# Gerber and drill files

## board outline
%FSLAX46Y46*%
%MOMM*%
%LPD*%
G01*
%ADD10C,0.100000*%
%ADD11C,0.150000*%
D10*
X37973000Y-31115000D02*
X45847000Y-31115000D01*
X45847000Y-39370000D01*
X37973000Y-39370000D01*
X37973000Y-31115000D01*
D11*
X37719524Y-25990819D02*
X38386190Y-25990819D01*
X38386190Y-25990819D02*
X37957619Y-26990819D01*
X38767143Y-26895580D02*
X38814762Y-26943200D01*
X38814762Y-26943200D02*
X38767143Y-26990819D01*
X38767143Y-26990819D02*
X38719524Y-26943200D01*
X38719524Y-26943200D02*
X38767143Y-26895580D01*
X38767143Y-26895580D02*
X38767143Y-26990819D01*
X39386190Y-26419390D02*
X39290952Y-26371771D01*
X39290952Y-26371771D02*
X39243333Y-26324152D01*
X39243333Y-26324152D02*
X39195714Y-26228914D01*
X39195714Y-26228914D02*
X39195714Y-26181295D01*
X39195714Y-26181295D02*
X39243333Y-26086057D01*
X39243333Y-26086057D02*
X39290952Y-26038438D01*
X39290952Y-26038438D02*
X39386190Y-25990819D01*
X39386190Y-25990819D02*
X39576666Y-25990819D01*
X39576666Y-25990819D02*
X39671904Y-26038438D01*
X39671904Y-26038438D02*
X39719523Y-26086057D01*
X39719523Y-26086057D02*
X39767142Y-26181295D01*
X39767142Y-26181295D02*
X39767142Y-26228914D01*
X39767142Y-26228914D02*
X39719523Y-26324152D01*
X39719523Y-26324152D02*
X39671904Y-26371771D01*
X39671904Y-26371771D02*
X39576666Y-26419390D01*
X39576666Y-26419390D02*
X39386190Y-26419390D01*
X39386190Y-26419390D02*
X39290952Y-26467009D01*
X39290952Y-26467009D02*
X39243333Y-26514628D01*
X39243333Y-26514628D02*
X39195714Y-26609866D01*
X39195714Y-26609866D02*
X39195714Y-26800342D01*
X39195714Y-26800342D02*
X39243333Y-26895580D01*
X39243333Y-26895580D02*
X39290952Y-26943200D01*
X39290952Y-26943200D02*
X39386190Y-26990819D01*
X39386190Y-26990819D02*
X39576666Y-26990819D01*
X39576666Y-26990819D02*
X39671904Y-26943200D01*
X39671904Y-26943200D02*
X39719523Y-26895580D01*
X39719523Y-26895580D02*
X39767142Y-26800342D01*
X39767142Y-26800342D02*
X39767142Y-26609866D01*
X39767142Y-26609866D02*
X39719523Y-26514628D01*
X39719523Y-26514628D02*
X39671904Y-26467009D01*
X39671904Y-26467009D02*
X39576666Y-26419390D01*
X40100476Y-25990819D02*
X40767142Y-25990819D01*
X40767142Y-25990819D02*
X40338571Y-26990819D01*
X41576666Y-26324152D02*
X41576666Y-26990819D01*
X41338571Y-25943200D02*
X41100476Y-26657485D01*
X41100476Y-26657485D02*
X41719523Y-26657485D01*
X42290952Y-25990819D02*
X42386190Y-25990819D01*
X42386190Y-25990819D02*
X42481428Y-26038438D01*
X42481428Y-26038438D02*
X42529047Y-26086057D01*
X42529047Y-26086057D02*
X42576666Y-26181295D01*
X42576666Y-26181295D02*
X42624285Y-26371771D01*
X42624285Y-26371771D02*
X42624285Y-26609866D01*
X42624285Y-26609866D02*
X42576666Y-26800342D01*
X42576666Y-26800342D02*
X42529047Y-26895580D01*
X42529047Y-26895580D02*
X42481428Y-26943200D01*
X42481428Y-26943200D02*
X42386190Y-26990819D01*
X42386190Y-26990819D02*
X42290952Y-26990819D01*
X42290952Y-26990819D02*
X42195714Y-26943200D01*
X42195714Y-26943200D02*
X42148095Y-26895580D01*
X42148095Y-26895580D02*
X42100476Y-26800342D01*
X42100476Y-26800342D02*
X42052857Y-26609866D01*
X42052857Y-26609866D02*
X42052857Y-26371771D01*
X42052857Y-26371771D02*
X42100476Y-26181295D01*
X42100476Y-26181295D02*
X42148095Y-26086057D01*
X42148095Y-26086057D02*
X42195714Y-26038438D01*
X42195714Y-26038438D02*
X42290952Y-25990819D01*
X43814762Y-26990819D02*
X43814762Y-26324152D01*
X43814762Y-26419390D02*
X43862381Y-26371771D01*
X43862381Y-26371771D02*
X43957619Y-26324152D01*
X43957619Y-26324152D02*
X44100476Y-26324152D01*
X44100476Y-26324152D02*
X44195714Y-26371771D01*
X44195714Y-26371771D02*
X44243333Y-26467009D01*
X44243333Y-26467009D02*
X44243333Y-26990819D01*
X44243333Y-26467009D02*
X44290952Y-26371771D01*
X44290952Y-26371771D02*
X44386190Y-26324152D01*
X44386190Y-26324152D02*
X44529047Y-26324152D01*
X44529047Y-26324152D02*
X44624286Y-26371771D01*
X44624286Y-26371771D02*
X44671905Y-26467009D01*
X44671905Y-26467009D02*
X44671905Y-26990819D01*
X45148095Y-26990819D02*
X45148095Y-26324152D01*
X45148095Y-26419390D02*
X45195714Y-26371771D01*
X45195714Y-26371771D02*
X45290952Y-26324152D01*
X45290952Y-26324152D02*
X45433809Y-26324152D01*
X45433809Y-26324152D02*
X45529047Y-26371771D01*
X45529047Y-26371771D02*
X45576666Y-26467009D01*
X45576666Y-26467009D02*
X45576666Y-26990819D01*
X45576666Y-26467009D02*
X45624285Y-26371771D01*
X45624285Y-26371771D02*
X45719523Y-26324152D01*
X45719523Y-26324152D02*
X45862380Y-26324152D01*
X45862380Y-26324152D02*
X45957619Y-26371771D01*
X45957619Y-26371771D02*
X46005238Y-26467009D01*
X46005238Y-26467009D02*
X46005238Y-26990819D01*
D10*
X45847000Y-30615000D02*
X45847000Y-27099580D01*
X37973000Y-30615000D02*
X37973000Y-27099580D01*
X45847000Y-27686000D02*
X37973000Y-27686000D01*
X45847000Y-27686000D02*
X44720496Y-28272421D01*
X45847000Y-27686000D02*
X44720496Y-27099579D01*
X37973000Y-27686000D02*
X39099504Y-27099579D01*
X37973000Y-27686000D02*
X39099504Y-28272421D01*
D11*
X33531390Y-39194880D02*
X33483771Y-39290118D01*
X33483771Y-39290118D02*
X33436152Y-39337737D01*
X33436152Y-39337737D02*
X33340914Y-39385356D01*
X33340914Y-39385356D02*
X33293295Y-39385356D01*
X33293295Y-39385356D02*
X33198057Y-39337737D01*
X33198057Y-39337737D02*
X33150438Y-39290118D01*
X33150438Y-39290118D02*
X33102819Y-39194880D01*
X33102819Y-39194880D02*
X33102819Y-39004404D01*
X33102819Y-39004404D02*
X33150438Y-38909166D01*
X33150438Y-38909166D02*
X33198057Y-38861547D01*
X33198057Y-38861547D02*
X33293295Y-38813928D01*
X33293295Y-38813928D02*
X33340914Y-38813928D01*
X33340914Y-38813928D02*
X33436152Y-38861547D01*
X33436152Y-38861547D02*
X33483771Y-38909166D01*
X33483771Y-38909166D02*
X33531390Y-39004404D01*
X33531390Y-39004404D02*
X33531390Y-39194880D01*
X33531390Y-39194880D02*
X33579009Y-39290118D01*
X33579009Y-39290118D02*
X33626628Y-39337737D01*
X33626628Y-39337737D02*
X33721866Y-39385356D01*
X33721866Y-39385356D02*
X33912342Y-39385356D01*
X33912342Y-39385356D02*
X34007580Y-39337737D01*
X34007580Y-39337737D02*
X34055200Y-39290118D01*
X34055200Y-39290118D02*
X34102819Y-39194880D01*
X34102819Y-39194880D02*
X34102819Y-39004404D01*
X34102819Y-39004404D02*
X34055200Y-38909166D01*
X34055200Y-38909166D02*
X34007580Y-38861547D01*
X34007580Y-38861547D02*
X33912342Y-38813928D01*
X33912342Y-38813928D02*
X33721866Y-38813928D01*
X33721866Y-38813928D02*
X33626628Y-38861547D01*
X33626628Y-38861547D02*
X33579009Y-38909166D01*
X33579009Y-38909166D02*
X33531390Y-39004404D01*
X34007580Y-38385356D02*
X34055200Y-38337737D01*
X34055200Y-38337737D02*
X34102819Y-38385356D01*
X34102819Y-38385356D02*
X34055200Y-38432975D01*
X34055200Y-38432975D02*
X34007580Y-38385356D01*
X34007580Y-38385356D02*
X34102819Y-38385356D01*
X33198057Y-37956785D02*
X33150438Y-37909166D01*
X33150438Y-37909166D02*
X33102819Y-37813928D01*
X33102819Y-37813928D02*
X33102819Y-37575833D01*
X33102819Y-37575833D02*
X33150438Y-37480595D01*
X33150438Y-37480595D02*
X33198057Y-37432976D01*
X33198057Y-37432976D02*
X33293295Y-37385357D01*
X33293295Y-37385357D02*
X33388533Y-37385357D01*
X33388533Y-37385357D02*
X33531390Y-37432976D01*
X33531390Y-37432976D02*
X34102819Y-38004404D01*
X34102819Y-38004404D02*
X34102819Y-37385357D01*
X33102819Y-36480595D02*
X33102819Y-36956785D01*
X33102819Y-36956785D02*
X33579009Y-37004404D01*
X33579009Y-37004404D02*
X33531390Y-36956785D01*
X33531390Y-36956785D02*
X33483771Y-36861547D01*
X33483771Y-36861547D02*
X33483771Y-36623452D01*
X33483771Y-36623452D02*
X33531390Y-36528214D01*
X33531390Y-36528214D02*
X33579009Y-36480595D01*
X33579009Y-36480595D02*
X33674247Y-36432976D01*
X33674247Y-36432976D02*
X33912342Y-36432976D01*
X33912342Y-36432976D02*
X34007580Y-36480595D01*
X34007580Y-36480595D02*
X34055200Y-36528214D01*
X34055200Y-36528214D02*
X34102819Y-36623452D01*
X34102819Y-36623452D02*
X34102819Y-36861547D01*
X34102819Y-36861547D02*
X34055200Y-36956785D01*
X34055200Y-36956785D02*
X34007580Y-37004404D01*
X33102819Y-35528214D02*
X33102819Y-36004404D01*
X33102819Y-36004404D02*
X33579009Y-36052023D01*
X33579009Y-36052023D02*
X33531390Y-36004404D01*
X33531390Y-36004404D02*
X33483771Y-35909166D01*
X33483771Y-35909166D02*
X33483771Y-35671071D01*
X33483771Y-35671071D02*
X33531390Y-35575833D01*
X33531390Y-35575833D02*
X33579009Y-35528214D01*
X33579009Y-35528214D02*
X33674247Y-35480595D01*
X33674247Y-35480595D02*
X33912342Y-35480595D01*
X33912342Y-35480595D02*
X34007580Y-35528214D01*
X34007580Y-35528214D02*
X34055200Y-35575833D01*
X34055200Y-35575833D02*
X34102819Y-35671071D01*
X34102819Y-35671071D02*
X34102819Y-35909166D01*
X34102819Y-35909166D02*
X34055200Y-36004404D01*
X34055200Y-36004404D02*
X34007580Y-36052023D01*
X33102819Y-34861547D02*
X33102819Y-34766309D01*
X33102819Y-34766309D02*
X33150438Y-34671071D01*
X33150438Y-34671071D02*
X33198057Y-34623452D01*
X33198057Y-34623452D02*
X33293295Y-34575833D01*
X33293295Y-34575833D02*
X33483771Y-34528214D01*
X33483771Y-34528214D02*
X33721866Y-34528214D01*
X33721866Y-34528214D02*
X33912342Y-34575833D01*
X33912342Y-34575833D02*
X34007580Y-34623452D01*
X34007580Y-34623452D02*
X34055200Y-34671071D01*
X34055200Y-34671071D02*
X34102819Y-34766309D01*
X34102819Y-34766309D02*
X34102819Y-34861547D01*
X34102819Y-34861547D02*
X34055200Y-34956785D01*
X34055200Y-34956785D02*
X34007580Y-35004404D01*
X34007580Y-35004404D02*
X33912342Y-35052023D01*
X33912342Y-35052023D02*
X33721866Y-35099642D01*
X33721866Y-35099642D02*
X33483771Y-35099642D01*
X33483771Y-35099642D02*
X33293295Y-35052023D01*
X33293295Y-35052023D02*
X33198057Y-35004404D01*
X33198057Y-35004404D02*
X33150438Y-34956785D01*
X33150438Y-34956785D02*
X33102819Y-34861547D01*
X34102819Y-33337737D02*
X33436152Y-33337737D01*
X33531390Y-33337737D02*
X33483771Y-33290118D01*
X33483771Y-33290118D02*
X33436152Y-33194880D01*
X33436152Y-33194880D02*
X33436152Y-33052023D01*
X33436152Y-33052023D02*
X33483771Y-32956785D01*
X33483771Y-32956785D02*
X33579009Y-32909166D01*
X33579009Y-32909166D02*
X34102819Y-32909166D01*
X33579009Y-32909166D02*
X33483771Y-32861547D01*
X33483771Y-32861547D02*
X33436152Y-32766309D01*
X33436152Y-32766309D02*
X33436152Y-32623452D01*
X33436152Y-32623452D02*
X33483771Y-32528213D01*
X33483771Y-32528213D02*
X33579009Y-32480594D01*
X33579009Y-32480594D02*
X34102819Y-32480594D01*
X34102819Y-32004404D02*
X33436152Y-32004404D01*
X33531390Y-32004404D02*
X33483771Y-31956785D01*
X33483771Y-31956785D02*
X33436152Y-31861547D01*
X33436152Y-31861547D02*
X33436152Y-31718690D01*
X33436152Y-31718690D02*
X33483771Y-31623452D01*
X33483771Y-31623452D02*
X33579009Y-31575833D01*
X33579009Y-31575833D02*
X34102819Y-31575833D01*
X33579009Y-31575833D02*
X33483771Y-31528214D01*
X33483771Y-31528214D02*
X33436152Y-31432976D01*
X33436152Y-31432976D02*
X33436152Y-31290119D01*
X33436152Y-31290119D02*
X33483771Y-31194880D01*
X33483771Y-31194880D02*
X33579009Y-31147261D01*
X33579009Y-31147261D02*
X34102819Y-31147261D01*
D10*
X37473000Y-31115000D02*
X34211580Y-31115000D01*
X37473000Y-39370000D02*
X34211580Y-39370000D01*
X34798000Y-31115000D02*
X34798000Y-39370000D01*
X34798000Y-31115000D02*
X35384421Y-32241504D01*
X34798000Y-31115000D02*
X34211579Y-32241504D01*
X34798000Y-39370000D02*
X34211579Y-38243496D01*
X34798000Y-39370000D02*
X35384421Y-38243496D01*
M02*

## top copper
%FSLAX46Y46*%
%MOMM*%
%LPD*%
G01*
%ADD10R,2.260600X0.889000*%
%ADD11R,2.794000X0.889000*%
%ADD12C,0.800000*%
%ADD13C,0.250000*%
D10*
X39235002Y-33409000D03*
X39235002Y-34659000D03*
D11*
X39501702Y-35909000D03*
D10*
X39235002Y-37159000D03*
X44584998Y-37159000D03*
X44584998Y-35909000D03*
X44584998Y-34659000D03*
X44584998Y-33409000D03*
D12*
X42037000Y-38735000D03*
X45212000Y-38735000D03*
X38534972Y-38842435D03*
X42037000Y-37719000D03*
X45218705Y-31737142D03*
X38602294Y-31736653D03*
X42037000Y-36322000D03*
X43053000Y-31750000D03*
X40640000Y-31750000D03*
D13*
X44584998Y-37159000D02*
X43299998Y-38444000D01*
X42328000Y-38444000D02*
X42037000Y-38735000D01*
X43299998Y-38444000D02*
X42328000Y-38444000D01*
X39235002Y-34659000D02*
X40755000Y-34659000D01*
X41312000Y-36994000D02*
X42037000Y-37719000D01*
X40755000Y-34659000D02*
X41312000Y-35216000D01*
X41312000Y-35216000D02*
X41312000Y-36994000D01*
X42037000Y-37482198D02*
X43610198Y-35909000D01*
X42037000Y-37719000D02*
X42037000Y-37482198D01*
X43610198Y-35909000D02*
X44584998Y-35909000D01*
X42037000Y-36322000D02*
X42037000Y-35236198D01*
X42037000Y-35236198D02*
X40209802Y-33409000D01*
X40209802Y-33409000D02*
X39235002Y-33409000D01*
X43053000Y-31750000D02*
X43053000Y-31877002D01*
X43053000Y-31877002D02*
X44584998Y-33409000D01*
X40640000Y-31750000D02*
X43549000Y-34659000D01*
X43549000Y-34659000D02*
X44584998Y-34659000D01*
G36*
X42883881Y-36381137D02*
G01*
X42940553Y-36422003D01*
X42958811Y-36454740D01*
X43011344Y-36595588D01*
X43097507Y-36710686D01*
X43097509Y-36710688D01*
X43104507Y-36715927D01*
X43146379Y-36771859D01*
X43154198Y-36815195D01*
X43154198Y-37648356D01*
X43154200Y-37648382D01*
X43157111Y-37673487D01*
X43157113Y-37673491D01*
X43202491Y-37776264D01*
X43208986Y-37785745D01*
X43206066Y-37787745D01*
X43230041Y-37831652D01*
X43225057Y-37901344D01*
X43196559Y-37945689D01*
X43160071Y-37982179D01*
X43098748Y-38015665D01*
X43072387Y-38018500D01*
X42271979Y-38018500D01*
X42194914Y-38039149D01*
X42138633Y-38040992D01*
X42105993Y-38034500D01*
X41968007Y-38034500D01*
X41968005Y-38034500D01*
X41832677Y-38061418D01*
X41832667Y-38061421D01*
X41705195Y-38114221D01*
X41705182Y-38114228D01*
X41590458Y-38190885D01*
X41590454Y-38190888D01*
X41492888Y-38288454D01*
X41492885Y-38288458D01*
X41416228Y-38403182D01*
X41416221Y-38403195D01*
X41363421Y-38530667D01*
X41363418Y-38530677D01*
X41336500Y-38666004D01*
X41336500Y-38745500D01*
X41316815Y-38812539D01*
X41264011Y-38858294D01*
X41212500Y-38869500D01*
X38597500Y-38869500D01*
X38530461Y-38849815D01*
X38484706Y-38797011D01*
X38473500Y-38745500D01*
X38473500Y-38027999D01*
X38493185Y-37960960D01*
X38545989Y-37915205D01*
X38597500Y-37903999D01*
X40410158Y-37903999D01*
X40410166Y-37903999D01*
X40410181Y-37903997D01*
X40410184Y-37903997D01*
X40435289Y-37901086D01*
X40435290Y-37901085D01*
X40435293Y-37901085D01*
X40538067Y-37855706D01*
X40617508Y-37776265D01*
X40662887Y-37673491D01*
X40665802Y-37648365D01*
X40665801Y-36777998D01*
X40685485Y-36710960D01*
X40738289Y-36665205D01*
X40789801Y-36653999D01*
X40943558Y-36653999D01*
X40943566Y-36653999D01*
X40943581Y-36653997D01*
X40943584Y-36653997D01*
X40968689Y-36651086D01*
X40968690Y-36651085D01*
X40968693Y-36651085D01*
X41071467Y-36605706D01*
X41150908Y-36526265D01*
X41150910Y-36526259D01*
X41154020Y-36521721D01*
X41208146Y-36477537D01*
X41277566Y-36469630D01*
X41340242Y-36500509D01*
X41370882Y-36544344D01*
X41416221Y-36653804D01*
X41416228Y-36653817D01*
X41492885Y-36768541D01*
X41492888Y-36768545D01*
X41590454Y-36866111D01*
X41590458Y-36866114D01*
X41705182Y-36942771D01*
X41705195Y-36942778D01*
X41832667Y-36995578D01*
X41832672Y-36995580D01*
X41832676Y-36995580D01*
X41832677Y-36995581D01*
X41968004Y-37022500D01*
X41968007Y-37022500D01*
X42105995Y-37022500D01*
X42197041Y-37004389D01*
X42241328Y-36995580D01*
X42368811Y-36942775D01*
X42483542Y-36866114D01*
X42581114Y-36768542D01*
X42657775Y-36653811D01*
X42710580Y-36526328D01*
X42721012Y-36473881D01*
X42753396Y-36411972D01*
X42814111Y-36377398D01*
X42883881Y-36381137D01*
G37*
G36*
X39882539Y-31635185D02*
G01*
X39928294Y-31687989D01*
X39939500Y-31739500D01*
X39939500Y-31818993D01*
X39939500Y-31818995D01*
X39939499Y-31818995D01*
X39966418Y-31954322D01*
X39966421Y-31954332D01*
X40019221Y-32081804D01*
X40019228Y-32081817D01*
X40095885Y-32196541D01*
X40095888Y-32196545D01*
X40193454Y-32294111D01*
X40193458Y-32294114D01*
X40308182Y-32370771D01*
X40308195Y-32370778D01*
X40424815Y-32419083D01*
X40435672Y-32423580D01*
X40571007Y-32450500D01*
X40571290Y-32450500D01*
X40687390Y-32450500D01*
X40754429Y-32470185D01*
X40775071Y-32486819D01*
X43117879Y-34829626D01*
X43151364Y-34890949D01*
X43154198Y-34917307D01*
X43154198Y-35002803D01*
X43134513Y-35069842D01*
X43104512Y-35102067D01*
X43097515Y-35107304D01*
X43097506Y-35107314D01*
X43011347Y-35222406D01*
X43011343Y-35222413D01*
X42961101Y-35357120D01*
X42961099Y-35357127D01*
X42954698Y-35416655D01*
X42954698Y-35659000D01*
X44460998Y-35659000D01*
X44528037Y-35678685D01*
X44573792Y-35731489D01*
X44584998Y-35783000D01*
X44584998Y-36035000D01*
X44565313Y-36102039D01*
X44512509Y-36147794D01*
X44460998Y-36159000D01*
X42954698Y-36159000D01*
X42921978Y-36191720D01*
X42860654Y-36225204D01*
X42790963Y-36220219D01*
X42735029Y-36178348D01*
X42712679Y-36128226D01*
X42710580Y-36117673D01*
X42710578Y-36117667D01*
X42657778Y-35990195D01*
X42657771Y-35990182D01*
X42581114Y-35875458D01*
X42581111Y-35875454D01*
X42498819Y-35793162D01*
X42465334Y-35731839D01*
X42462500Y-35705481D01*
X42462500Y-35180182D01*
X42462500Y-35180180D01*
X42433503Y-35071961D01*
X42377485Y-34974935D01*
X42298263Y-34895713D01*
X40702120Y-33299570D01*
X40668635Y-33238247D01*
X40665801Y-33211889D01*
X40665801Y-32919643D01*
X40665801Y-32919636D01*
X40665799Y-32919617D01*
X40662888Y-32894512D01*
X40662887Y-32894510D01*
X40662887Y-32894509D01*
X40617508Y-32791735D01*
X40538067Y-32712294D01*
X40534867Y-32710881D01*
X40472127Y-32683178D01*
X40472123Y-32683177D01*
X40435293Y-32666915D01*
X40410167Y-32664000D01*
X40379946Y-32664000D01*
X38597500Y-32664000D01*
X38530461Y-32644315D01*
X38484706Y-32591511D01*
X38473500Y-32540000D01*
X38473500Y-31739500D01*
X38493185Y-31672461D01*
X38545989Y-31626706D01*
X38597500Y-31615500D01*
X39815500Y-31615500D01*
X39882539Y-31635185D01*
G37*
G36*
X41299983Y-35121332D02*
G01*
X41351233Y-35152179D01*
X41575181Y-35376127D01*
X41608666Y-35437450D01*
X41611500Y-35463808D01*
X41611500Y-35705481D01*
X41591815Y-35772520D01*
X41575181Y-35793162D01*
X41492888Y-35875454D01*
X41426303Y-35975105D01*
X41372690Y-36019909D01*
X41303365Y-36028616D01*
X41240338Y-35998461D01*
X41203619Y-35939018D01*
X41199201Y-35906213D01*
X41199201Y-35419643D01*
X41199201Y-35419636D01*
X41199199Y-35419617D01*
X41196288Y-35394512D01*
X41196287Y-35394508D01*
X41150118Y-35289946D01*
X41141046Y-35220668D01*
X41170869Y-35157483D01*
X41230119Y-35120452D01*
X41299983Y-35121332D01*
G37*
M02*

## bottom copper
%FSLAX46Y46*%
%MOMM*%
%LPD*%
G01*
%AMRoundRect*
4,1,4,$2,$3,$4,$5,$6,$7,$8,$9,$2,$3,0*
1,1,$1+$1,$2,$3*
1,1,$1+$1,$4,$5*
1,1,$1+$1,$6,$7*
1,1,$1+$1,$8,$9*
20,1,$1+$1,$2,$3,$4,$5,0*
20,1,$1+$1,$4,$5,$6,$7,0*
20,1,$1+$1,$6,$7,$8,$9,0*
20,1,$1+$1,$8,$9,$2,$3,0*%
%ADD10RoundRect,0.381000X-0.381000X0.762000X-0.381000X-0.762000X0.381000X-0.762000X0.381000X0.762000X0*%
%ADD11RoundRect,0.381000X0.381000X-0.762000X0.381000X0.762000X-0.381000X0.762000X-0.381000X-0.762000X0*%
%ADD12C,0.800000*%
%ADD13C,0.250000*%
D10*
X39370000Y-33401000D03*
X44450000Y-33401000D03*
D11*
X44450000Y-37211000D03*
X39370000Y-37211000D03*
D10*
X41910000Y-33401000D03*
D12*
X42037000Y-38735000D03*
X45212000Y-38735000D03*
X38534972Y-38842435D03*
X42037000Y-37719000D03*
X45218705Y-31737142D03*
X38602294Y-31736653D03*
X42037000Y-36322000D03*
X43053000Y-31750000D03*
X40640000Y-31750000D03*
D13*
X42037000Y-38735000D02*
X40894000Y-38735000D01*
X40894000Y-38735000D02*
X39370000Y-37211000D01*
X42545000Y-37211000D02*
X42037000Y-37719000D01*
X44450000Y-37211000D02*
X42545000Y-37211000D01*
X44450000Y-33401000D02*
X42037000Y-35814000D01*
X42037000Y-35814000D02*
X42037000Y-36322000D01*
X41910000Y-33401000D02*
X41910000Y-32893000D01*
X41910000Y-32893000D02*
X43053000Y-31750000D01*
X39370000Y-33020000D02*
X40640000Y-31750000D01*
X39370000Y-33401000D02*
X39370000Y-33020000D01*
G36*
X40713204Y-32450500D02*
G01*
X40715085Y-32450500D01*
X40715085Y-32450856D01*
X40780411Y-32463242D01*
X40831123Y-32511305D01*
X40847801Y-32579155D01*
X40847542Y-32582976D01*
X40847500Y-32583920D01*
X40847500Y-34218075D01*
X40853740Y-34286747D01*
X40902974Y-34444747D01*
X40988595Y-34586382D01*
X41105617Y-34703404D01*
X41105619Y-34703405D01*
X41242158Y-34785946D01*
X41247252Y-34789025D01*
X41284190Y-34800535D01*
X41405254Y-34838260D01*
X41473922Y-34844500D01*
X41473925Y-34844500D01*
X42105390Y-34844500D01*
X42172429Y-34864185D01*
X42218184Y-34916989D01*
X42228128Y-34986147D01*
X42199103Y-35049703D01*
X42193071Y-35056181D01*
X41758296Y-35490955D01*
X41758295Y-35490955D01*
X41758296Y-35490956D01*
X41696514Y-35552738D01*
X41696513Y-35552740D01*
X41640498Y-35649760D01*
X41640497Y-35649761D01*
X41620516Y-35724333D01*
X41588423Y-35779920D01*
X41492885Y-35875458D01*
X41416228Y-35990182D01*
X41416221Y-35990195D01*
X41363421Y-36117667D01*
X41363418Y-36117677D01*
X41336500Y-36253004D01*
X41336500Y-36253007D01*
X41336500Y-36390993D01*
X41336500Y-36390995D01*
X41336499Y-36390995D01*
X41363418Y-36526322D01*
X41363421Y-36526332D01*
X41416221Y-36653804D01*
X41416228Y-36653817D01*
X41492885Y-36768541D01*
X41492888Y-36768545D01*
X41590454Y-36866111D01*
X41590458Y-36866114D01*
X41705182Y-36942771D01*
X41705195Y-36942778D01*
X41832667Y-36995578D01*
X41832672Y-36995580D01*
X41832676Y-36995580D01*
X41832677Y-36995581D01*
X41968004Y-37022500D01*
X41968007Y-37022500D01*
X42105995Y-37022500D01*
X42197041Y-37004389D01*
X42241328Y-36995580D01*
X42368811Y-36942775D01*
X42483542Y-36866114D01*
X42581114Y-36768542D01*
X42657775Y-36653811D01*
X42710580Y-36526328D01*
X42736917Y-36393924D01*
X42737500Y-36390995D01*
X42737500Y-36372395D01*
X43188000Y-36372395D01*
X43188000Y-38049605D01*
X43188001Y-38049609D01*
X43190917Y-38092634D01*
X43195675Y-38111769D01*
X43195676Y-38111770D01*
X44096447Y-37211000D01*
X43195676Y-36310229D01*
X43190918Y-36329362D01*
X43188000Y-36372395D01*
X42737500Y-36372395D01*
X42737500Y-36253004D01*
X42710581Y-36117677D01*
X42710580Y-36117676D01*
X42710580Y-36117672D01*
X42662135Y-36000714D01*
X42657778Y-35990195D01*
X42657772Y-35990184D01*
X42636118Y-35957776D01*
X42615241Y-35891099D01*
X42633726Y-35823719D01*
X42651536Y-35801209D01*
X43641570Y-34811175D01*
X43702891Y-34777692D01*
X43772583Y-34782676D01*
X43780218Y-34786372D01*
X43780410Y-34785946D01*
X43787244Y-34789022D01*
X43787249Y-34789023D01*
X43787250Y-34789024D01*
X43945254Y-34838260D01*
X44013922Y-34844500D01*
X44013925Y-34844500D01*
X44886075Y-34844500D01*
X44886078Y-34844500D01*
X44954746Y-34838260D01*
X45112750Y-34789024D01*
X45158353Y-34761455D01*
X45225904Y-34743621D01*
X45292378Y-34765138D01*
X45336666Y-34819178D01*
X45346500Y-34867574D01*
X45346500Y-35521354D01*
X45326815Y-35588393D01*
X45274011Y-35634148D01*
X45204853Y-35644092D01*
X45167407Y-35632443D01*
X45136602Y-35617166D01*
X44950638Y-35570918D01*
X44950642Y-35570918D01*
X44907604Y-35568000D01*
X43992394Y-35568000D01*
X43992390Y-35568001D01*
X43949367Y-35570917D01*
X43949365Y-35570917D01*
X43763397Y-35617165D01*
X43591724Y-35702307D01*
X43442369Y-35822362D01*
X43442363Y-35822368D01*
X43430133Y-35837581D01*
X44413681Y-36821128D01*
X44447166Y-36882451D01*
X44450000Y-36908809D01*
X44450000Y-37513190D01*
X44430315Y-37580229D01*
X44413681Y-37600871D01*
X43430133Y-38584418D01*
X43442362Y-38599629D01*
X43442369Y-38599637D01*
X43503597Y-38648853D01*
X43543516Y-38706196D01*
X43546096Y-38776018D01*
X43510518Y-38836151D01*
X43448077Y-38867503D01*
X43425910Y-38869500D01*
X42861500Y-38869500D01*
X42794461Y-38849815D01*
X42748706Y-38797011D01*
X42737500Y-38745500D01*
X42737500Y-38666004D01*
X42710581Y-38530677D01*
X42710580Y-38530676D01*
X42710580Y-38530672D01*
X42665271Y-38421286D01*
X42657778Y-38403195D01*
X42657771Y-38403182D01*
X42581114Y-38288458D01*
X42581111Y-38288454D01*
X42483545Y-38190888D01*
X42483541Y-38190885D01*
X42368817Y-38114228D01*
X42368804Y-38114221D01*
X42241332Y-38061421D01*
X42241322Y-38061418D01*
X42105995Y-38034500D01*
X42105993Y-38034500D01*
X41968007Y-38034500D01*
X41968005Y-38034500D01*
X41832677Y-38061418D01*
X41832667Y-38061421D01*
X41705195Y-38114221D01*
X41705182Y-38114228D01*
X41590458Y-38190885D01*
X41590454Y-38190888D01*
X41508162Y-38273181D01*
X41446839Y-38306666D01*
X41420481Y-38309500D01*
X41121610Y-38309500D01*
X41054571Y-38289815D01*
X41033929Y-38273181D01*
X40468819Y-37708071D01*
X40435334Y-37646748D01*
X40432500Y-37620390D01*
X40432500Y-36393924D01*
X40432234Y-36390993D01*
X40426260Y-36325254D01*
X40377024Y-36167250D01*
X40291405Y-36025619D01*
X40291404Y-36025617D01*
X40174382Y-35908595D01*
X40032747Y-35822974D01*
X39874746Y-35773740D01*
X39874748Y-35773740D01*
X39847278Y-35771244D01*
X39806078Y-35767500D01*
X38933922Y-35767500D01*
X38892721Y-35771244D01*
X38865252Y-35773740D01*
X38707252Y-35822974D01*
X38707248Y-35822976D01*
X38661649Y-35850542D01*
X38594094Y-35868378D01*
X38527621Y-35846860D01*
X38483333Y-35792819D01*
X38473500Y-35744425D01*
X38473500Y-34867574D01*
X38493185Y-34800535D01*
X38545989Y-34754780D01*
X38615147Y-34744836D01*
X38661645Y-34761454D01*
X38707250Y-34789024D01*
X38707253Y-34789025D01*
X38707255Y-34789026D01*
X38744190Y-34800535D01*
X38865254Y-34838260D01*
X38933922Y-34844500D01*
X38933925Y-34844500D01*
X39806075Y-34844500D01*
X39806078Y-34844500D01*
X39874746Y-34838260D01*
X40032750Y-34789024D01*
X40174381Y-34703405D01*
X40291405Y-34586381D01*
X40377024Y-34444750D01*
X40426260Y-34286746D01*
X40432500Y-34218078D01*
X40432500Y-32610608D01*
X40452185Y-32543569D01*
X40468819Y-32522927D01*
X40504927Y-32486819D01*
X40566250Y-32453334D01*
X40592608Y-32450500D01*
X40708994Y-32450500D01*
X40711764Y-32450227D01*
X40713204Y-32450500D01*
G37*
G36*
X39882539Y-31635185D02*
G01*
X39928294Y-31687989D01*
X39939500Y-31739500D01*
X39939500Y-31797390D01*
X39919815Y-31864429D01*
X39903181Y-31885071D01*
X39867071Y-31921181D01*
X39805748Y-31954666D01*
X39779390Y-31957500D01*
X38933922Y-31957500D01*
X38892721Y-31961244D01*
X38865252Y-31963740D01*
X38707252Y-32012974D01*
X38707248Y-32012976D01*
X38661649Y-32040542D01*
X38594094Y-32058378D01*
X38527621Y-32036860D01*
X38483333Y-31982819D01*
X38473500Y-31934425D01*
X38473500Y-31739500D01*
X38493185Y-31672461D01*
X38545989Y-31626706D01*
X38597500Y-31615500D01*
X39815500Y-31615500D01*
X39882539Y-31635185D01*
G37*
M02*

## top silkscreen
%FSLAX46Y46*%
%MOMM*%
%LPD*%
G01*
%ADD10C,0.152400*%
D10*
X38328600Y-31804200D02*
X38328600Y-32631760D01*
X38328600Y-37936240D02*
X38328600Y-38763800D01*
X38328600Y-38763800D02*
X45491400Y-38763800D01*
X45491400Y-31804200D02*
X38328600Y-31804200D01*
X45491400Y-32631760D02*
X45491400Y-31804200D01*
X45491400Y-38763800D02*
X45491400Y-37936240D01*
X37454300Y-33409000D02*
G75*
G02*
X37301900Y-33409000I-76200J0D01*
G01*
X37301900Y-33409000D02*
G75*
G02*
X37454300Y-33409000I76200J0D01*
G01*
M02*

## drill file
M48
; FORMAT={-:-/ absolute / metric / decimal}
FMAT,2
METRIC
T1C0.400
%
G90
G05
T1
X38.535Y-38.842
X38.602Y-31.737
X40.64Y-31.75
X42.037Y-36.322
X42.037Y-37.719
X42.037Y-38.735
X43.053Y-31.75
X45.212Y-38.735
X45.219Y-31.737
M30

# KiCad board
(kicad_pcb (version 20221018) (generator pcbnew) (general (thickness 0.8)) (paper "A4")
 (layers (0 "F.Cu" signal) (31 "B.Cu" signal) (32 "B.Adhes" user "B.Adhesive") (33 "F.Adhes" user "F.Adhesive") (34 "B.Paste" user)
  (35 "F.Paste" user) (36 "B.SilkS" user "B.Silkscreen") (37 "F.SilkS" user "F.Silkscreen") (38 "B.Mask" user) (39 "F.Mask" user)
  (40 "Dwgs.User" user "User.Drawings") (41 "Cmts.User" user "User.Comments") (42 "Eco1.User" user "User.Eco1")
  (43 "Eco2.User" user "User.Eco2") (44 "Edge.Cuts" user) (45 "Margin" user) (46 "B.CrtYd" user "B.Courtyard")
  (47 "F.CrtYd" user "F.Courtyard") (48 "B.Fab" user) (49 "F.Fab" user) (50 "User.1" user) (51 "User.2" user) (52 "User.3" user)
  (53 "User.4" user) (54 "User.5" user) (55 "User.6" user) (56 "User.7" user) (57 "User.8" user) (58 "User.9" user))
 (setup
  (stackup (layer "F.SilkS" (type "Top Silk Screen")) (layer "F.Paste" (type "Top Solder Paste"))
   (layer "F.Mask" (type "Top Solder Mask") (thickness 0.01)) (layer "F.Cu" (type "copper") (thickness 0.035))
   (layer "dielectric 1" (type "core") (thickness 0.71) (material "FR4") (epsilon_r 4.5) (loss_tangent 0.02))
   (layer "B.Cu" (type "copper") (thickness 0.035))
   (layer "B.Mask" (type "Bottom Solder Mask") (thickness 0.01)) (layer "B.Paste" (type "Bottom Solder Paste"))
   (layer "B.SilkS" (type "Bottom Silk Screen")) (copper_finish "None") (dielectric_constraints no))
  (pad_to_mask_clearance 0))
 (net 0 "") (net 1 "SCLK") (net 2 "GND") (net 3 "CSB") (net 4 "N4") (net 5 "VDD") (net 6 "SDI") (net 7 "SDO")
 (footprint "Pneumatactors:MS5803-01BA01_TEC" (layer "F.Cu") (at 41.91 35.284)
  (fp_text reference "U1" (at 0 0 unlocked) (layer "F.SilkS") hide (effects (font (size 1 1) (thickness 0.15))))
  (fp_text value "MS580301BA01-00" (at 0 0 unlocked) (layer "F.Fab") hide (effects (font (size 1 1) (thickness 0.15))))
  (fp_line (start -3.5814 -3.4798) (end -3.5814 -2.65224) (stroke (width 0.1524) (type solid)) (layer "F.SilkS"))
  (fp_line (start -3.5814 2.65224) (end -3.5814 3.4798) (stroke (width 0.1524) (type solid)) (layer "F.SilkS"))
  (fp_line (start -3.5814 3.4798) (end 3.5814 3.4798) (stroke (width 0.1524) (type solid)) (layer "F.SilkS"))
  (fp_line (start 3.5814 -3.4798) (end -3.5814 -3.4798) (stroke (width 0.1524) (type solid)) (layer "F.SilkS"))
  (fp_line (start 3.5814 -2.65224) (end 3.5814 -3.4798) (stroke (width 0.1524) (type solid)) (layer "F.SilkS"))
  (fp_line (start 3.5814 3.4798) (end 3.5814 2.65224) (stroke (width 0.1524) (type solid)) (layer "F.SilkS"))
  (fp_circle (center -4.5319 -1.875) (end -4.4557 -1.875) (stroke (width 0.1524) (type solid)) (fill none) (layer "F.SilkS"))
  (pad "1" smd rect (at -2.674998 -1.875) (size 2.2606 0.889) (layers "F.Cu" "F.Paste" "F.Mask") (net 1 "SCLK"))
  (pad "2" smd rect (at -2.674998 -0.625) (size 2.2606 0.889) (layers "F.Cu" "F.Paste" "F.Mask") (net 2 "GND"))
  (pad "3" smd rect (at -2.408298 0.625) (size 2.794 0.889) (layers "F.Cu" "F.Paste" "F.Mask") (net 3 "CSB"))
  (pad "4" smd rect (at -2.674998 1.875) (size 2.2606 0.889) (layers "F.Cu" "F.Paste" "F.Mask") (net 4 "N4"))
  (pad "5" smd rect (at 2.674998 1.875) (size 2.2606 0.889) (layers "F.Cu" "F.Paste" "F.Mask") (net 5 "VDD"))
  (pad "6" smd rect (at 2.674998 0.625) (size 2.2606 0.889) (layers "F.Cu" "F.Paste" "F.Mask") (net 2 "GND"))
  (pad "7" smd rect (at 2.674998 -0.625) (size 2.2606 0.889) (layers "F.Cu" "F.Paste" "F.Mask") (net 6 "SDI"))
  (pad "8" smd rect (at 2.674998 -1.875) (size 2.2606 0.889) (layers "F.Cu" "F.Paste" "F.Mask") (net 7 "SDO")))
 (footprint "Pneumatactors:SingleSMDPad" (layer "B.Cu") (at 41.91 33.401 -90)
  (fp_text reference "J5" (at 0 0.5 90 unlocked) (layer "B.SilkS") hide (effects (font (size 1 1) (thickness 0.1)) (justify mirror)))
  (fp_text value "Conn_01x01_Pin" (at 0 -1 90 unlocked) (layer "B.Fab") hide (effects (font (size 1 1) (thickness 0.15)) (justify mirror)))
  (pad "1" smd roundrect (at 0 2.54 270) (size 2.286 1.524) (layers "B.Cu" "B.Paste" "B.Mask") (roundrect_rratio 0.25) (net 6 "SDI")
   (thermal_bridge_angle 45)))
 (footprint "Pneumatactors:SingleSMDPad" (layer "B.Cu") (at 46.99 33.401 -90)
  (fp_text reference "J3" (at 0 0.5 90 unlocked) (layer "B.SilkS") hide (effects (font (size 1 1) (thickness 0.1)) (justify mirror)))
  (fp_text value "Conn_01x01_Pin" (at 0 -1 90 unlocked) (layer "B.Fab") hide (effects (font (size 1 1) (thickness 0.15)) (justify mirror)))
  (pad "1" smd roundrect (at 0 2.54 270) (size 2.286 1.524) (layers "B.Cu" "B.Paste" "B.Mask") (roundrect_rratio 0.25) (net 1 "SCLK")
   (thermal_bridge_angle 45)))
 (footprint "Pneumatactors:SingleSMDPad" (layer "B.Cu") (at 41.91 37.211 90)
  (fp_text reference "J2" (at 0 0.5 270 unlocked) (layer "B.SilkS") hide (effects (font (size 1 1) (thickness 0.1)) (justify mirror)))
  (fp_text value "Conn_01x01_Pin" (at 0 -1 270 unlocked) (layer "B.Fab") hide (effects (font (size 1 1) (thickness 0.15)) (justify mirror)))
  (pad "1" smd roundrect (at 0 2.54 90) (size 2.286 1.524) (layers "B.Cu" "B.Paste" "B.Mask") (roundrect_rratio 0.25) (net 2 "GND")
   (thermal_bridge_angle 45)))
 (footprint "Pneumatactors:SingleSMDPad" (layer "B.Cu") (at 36.83 37.211 90)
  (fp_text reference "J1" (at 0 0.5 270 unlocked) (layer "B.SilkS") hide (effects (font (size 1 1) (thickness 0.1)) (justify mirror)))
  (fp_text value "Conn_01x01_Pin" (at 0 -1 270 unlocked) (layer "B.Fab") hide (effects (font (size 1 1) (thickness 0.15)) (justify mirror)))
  (pad "1" smd roundrect (at 0 2.54 90) (size 2.286 1.524) (layers "B.Cu" "B.Paste" "B.Mask") (roundrect_rratio 0.25) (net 5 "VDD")
   (thermal_bridge_angle 45)))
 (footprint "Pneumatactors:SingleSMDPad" (layer "B.Cu") (at 44.45 33.401 -90)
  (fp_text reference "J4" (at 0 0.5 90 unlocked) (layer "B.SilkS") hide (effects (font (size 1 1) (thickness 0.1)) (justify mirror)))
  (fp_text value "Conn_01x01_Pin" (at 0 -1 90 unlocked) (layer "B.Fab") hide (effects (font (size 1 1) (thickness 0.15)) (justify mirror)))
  (pad "1" smd roundrect (at 0 2.54 270) (size 2.286 1.524) (layers "B.Cu" "B.Paste" "B.Mask") (roundrect_rratio 0.25) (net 7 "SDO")
   (thermal_bridge_angle 45)))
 (gr_rect (start 37.973 31.115) (end 45.847 39.37) (stroke (width 0.1) (type default)) (fill none) (layer "Edge.Cuts"))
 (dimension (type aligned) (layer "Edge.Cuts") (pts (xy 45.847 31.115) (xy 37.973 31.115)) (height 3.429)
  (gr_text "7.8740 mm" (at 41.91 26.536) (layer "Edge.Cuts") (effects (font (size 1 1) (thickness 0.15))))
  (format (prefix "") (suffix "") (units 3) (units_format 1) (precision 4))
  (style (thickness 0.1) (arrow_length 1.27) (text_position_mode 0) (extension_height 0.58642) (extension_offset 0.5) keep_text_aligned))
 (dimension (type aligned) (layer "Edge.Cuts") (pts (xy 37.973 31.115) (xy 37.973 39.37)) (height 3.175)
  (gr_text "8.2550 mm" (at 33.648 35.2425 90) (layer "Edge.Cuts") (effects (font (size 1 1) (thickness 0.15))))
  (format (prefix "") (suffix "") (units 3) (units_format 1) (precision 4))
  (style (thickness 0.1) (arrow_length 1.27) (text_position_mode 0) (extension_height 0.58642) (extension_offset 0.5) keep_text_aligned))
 (segment (start 44.584998 37.159) (end 43.299998 38.444) (width 0.25) (layer "F.Cu") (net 5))
 (segment (start 42.328 38.444) (end 42.037 38.735) (width 0.25) (layer "F.Cu") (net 5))
 (segment (start 43.299998 38.444) (end 42.328 38.444) (width 0.25) (layer "F.Cu") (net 5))
 (via (at 42.037 38.735) (size 0.8) (drill 0.4) (layers "F.Cu" "B.Cu") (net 5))
 (segment (start 42.037 38.735) (end 40.894 38.735) (width 0.25) (layer "B.Cu") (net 5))
 (segment (start 40.894 38.735) (end 39.37 37.211) (width 0.25) (layer "B.Cu") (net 5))
 (segment (start 39.235002 34.659) (end 40.755 34.659) (width 0.25) (layer "F.Cu") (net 2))
 (segment (start 41.312 36.994) (end 42.037 37.719) (width 0.25) (layer "F.Cu") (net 2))
 (segment (start 40.755 34.659) (end 41.312 35.216) (width 0.25) (layer "F.Cu") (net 2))
 (segment (start 41.312 35.216) (end 41.312 36.994) (width 0.25) (layer "F.Cu") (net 2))
 (segment (start 42.037 37.482198) (end 43.610198 35.909) (width 0.25) (layer "F.Cu") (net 2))
 (segment (start 42.037 37.719) (end 42.037 37.482198) (width 0.25) (layer "F.Cu") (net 2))
 (segment (start 43.610198 35.909) (end 44.584998 35.909) (width 0.25) (layer "F.Cu") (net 2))
 (via (at 45.212 38.735) (size 0.8) (drill 0.4) (layers "F.Cu" "B.Cu") (free) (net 2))
 (via (at 38.534972 38.842435) (size 0.8) (drill 0.4) (layers "F.Cu" "B.Cu") (free) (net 2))
 (via (at 42.037 37.719) (size 0.8) (drill 0.4) (layers "F.Cu" "B.Cu") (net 2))
 (via (at 45.218705 31.737142) (size 0.8) (drill 0.4) (layers "F.Cu" "B.Cu") (free) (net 2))
 (via (at 38.602294 31.736653) (size 0.8) (drill 0.4) (layers "F.Cu" "B.Cu") (free) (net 2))
 (segment (start 42.545 37.211) (end 42.037 37.719) (width 0.25) (layer "B.Cu") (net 2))
 (segment (start 44.45 37.211) (end 42.545 37.211) (width 0.25) (layer "B.Cu") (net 2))
 (segment (start 42.037 36.322) (end 42.037 35.236198) (width 0.25) (layer "F.Cu") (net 1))
 (segment (start 42.037 35.236198) (end 40.209802 33.409) (width 0.25) (layer "F.Cu") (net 1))
 (segment (start 40.209802 33.409) (end 39.235002 33.409) (width 0.25) (layer "F.Cu") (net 1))
 (via (at 42.037 36.322) (size 0.8) (drill 0.4) (layers "F.Cu" "B.Cu") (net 1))
 (segment (start 44.45 33.401) (end 42.037 35.814) (width 0.25) (layer "B.Cu") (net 1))
 (segment (start 42.037 35.814) (end 42.037 36.322) (width 0.25) (layer "B.Cu") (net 1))
 (segment (start 43.053 31.75) (end 43.053 31.877002) (width 0.25) (layer "F.Cu") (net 7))
 (segment (start 43.053 31.877002) (end 44.584998 33.409) (width 0.25) (layer "F.Cu") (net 7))
 (via (at 43.053 31.75) (size 0.8) (drill 0.4) (layers "F.Cu" "B.Cu") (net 7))
 (segment (start 41.91 33.401) (end 41.91 32.893) (width 0.25) (layer "B.Cu") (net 7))
 (segment (start 41.91 32.893) (end 43.053 31.75) (width 0.25) (layer "B.Cu") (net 7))
 (segment (start 40.64 31.75) (end 43.549 34.659) (width 0.25) (layer "F.Cu") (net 6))
 (segment (start 43.549 34.659) (end 44.584998 34.659) (width 0.25) (layer "F.Cu") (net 6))
 (via (at 40.64 31.75) (size 0.8) (drill 0.4) (layers "F.Cu" "B.Cu") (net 6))
 (segment (start 39.37 33.02) (end 40.64 31.75) (width 0.25) (layer "B.Cu") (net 6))
 (segment (start 39.37 33.401) (end 39.37 33.02) (width 0.25) (layer "B.Cu") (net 6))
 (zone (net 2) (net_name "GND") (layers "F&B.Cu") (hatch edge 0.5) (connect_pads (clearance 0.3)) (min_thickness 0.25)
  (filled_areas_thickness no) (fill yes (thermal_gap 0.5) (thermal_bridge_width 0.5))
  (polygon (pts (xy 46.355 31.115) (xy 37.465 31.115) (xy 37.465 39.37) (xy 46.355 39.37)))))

